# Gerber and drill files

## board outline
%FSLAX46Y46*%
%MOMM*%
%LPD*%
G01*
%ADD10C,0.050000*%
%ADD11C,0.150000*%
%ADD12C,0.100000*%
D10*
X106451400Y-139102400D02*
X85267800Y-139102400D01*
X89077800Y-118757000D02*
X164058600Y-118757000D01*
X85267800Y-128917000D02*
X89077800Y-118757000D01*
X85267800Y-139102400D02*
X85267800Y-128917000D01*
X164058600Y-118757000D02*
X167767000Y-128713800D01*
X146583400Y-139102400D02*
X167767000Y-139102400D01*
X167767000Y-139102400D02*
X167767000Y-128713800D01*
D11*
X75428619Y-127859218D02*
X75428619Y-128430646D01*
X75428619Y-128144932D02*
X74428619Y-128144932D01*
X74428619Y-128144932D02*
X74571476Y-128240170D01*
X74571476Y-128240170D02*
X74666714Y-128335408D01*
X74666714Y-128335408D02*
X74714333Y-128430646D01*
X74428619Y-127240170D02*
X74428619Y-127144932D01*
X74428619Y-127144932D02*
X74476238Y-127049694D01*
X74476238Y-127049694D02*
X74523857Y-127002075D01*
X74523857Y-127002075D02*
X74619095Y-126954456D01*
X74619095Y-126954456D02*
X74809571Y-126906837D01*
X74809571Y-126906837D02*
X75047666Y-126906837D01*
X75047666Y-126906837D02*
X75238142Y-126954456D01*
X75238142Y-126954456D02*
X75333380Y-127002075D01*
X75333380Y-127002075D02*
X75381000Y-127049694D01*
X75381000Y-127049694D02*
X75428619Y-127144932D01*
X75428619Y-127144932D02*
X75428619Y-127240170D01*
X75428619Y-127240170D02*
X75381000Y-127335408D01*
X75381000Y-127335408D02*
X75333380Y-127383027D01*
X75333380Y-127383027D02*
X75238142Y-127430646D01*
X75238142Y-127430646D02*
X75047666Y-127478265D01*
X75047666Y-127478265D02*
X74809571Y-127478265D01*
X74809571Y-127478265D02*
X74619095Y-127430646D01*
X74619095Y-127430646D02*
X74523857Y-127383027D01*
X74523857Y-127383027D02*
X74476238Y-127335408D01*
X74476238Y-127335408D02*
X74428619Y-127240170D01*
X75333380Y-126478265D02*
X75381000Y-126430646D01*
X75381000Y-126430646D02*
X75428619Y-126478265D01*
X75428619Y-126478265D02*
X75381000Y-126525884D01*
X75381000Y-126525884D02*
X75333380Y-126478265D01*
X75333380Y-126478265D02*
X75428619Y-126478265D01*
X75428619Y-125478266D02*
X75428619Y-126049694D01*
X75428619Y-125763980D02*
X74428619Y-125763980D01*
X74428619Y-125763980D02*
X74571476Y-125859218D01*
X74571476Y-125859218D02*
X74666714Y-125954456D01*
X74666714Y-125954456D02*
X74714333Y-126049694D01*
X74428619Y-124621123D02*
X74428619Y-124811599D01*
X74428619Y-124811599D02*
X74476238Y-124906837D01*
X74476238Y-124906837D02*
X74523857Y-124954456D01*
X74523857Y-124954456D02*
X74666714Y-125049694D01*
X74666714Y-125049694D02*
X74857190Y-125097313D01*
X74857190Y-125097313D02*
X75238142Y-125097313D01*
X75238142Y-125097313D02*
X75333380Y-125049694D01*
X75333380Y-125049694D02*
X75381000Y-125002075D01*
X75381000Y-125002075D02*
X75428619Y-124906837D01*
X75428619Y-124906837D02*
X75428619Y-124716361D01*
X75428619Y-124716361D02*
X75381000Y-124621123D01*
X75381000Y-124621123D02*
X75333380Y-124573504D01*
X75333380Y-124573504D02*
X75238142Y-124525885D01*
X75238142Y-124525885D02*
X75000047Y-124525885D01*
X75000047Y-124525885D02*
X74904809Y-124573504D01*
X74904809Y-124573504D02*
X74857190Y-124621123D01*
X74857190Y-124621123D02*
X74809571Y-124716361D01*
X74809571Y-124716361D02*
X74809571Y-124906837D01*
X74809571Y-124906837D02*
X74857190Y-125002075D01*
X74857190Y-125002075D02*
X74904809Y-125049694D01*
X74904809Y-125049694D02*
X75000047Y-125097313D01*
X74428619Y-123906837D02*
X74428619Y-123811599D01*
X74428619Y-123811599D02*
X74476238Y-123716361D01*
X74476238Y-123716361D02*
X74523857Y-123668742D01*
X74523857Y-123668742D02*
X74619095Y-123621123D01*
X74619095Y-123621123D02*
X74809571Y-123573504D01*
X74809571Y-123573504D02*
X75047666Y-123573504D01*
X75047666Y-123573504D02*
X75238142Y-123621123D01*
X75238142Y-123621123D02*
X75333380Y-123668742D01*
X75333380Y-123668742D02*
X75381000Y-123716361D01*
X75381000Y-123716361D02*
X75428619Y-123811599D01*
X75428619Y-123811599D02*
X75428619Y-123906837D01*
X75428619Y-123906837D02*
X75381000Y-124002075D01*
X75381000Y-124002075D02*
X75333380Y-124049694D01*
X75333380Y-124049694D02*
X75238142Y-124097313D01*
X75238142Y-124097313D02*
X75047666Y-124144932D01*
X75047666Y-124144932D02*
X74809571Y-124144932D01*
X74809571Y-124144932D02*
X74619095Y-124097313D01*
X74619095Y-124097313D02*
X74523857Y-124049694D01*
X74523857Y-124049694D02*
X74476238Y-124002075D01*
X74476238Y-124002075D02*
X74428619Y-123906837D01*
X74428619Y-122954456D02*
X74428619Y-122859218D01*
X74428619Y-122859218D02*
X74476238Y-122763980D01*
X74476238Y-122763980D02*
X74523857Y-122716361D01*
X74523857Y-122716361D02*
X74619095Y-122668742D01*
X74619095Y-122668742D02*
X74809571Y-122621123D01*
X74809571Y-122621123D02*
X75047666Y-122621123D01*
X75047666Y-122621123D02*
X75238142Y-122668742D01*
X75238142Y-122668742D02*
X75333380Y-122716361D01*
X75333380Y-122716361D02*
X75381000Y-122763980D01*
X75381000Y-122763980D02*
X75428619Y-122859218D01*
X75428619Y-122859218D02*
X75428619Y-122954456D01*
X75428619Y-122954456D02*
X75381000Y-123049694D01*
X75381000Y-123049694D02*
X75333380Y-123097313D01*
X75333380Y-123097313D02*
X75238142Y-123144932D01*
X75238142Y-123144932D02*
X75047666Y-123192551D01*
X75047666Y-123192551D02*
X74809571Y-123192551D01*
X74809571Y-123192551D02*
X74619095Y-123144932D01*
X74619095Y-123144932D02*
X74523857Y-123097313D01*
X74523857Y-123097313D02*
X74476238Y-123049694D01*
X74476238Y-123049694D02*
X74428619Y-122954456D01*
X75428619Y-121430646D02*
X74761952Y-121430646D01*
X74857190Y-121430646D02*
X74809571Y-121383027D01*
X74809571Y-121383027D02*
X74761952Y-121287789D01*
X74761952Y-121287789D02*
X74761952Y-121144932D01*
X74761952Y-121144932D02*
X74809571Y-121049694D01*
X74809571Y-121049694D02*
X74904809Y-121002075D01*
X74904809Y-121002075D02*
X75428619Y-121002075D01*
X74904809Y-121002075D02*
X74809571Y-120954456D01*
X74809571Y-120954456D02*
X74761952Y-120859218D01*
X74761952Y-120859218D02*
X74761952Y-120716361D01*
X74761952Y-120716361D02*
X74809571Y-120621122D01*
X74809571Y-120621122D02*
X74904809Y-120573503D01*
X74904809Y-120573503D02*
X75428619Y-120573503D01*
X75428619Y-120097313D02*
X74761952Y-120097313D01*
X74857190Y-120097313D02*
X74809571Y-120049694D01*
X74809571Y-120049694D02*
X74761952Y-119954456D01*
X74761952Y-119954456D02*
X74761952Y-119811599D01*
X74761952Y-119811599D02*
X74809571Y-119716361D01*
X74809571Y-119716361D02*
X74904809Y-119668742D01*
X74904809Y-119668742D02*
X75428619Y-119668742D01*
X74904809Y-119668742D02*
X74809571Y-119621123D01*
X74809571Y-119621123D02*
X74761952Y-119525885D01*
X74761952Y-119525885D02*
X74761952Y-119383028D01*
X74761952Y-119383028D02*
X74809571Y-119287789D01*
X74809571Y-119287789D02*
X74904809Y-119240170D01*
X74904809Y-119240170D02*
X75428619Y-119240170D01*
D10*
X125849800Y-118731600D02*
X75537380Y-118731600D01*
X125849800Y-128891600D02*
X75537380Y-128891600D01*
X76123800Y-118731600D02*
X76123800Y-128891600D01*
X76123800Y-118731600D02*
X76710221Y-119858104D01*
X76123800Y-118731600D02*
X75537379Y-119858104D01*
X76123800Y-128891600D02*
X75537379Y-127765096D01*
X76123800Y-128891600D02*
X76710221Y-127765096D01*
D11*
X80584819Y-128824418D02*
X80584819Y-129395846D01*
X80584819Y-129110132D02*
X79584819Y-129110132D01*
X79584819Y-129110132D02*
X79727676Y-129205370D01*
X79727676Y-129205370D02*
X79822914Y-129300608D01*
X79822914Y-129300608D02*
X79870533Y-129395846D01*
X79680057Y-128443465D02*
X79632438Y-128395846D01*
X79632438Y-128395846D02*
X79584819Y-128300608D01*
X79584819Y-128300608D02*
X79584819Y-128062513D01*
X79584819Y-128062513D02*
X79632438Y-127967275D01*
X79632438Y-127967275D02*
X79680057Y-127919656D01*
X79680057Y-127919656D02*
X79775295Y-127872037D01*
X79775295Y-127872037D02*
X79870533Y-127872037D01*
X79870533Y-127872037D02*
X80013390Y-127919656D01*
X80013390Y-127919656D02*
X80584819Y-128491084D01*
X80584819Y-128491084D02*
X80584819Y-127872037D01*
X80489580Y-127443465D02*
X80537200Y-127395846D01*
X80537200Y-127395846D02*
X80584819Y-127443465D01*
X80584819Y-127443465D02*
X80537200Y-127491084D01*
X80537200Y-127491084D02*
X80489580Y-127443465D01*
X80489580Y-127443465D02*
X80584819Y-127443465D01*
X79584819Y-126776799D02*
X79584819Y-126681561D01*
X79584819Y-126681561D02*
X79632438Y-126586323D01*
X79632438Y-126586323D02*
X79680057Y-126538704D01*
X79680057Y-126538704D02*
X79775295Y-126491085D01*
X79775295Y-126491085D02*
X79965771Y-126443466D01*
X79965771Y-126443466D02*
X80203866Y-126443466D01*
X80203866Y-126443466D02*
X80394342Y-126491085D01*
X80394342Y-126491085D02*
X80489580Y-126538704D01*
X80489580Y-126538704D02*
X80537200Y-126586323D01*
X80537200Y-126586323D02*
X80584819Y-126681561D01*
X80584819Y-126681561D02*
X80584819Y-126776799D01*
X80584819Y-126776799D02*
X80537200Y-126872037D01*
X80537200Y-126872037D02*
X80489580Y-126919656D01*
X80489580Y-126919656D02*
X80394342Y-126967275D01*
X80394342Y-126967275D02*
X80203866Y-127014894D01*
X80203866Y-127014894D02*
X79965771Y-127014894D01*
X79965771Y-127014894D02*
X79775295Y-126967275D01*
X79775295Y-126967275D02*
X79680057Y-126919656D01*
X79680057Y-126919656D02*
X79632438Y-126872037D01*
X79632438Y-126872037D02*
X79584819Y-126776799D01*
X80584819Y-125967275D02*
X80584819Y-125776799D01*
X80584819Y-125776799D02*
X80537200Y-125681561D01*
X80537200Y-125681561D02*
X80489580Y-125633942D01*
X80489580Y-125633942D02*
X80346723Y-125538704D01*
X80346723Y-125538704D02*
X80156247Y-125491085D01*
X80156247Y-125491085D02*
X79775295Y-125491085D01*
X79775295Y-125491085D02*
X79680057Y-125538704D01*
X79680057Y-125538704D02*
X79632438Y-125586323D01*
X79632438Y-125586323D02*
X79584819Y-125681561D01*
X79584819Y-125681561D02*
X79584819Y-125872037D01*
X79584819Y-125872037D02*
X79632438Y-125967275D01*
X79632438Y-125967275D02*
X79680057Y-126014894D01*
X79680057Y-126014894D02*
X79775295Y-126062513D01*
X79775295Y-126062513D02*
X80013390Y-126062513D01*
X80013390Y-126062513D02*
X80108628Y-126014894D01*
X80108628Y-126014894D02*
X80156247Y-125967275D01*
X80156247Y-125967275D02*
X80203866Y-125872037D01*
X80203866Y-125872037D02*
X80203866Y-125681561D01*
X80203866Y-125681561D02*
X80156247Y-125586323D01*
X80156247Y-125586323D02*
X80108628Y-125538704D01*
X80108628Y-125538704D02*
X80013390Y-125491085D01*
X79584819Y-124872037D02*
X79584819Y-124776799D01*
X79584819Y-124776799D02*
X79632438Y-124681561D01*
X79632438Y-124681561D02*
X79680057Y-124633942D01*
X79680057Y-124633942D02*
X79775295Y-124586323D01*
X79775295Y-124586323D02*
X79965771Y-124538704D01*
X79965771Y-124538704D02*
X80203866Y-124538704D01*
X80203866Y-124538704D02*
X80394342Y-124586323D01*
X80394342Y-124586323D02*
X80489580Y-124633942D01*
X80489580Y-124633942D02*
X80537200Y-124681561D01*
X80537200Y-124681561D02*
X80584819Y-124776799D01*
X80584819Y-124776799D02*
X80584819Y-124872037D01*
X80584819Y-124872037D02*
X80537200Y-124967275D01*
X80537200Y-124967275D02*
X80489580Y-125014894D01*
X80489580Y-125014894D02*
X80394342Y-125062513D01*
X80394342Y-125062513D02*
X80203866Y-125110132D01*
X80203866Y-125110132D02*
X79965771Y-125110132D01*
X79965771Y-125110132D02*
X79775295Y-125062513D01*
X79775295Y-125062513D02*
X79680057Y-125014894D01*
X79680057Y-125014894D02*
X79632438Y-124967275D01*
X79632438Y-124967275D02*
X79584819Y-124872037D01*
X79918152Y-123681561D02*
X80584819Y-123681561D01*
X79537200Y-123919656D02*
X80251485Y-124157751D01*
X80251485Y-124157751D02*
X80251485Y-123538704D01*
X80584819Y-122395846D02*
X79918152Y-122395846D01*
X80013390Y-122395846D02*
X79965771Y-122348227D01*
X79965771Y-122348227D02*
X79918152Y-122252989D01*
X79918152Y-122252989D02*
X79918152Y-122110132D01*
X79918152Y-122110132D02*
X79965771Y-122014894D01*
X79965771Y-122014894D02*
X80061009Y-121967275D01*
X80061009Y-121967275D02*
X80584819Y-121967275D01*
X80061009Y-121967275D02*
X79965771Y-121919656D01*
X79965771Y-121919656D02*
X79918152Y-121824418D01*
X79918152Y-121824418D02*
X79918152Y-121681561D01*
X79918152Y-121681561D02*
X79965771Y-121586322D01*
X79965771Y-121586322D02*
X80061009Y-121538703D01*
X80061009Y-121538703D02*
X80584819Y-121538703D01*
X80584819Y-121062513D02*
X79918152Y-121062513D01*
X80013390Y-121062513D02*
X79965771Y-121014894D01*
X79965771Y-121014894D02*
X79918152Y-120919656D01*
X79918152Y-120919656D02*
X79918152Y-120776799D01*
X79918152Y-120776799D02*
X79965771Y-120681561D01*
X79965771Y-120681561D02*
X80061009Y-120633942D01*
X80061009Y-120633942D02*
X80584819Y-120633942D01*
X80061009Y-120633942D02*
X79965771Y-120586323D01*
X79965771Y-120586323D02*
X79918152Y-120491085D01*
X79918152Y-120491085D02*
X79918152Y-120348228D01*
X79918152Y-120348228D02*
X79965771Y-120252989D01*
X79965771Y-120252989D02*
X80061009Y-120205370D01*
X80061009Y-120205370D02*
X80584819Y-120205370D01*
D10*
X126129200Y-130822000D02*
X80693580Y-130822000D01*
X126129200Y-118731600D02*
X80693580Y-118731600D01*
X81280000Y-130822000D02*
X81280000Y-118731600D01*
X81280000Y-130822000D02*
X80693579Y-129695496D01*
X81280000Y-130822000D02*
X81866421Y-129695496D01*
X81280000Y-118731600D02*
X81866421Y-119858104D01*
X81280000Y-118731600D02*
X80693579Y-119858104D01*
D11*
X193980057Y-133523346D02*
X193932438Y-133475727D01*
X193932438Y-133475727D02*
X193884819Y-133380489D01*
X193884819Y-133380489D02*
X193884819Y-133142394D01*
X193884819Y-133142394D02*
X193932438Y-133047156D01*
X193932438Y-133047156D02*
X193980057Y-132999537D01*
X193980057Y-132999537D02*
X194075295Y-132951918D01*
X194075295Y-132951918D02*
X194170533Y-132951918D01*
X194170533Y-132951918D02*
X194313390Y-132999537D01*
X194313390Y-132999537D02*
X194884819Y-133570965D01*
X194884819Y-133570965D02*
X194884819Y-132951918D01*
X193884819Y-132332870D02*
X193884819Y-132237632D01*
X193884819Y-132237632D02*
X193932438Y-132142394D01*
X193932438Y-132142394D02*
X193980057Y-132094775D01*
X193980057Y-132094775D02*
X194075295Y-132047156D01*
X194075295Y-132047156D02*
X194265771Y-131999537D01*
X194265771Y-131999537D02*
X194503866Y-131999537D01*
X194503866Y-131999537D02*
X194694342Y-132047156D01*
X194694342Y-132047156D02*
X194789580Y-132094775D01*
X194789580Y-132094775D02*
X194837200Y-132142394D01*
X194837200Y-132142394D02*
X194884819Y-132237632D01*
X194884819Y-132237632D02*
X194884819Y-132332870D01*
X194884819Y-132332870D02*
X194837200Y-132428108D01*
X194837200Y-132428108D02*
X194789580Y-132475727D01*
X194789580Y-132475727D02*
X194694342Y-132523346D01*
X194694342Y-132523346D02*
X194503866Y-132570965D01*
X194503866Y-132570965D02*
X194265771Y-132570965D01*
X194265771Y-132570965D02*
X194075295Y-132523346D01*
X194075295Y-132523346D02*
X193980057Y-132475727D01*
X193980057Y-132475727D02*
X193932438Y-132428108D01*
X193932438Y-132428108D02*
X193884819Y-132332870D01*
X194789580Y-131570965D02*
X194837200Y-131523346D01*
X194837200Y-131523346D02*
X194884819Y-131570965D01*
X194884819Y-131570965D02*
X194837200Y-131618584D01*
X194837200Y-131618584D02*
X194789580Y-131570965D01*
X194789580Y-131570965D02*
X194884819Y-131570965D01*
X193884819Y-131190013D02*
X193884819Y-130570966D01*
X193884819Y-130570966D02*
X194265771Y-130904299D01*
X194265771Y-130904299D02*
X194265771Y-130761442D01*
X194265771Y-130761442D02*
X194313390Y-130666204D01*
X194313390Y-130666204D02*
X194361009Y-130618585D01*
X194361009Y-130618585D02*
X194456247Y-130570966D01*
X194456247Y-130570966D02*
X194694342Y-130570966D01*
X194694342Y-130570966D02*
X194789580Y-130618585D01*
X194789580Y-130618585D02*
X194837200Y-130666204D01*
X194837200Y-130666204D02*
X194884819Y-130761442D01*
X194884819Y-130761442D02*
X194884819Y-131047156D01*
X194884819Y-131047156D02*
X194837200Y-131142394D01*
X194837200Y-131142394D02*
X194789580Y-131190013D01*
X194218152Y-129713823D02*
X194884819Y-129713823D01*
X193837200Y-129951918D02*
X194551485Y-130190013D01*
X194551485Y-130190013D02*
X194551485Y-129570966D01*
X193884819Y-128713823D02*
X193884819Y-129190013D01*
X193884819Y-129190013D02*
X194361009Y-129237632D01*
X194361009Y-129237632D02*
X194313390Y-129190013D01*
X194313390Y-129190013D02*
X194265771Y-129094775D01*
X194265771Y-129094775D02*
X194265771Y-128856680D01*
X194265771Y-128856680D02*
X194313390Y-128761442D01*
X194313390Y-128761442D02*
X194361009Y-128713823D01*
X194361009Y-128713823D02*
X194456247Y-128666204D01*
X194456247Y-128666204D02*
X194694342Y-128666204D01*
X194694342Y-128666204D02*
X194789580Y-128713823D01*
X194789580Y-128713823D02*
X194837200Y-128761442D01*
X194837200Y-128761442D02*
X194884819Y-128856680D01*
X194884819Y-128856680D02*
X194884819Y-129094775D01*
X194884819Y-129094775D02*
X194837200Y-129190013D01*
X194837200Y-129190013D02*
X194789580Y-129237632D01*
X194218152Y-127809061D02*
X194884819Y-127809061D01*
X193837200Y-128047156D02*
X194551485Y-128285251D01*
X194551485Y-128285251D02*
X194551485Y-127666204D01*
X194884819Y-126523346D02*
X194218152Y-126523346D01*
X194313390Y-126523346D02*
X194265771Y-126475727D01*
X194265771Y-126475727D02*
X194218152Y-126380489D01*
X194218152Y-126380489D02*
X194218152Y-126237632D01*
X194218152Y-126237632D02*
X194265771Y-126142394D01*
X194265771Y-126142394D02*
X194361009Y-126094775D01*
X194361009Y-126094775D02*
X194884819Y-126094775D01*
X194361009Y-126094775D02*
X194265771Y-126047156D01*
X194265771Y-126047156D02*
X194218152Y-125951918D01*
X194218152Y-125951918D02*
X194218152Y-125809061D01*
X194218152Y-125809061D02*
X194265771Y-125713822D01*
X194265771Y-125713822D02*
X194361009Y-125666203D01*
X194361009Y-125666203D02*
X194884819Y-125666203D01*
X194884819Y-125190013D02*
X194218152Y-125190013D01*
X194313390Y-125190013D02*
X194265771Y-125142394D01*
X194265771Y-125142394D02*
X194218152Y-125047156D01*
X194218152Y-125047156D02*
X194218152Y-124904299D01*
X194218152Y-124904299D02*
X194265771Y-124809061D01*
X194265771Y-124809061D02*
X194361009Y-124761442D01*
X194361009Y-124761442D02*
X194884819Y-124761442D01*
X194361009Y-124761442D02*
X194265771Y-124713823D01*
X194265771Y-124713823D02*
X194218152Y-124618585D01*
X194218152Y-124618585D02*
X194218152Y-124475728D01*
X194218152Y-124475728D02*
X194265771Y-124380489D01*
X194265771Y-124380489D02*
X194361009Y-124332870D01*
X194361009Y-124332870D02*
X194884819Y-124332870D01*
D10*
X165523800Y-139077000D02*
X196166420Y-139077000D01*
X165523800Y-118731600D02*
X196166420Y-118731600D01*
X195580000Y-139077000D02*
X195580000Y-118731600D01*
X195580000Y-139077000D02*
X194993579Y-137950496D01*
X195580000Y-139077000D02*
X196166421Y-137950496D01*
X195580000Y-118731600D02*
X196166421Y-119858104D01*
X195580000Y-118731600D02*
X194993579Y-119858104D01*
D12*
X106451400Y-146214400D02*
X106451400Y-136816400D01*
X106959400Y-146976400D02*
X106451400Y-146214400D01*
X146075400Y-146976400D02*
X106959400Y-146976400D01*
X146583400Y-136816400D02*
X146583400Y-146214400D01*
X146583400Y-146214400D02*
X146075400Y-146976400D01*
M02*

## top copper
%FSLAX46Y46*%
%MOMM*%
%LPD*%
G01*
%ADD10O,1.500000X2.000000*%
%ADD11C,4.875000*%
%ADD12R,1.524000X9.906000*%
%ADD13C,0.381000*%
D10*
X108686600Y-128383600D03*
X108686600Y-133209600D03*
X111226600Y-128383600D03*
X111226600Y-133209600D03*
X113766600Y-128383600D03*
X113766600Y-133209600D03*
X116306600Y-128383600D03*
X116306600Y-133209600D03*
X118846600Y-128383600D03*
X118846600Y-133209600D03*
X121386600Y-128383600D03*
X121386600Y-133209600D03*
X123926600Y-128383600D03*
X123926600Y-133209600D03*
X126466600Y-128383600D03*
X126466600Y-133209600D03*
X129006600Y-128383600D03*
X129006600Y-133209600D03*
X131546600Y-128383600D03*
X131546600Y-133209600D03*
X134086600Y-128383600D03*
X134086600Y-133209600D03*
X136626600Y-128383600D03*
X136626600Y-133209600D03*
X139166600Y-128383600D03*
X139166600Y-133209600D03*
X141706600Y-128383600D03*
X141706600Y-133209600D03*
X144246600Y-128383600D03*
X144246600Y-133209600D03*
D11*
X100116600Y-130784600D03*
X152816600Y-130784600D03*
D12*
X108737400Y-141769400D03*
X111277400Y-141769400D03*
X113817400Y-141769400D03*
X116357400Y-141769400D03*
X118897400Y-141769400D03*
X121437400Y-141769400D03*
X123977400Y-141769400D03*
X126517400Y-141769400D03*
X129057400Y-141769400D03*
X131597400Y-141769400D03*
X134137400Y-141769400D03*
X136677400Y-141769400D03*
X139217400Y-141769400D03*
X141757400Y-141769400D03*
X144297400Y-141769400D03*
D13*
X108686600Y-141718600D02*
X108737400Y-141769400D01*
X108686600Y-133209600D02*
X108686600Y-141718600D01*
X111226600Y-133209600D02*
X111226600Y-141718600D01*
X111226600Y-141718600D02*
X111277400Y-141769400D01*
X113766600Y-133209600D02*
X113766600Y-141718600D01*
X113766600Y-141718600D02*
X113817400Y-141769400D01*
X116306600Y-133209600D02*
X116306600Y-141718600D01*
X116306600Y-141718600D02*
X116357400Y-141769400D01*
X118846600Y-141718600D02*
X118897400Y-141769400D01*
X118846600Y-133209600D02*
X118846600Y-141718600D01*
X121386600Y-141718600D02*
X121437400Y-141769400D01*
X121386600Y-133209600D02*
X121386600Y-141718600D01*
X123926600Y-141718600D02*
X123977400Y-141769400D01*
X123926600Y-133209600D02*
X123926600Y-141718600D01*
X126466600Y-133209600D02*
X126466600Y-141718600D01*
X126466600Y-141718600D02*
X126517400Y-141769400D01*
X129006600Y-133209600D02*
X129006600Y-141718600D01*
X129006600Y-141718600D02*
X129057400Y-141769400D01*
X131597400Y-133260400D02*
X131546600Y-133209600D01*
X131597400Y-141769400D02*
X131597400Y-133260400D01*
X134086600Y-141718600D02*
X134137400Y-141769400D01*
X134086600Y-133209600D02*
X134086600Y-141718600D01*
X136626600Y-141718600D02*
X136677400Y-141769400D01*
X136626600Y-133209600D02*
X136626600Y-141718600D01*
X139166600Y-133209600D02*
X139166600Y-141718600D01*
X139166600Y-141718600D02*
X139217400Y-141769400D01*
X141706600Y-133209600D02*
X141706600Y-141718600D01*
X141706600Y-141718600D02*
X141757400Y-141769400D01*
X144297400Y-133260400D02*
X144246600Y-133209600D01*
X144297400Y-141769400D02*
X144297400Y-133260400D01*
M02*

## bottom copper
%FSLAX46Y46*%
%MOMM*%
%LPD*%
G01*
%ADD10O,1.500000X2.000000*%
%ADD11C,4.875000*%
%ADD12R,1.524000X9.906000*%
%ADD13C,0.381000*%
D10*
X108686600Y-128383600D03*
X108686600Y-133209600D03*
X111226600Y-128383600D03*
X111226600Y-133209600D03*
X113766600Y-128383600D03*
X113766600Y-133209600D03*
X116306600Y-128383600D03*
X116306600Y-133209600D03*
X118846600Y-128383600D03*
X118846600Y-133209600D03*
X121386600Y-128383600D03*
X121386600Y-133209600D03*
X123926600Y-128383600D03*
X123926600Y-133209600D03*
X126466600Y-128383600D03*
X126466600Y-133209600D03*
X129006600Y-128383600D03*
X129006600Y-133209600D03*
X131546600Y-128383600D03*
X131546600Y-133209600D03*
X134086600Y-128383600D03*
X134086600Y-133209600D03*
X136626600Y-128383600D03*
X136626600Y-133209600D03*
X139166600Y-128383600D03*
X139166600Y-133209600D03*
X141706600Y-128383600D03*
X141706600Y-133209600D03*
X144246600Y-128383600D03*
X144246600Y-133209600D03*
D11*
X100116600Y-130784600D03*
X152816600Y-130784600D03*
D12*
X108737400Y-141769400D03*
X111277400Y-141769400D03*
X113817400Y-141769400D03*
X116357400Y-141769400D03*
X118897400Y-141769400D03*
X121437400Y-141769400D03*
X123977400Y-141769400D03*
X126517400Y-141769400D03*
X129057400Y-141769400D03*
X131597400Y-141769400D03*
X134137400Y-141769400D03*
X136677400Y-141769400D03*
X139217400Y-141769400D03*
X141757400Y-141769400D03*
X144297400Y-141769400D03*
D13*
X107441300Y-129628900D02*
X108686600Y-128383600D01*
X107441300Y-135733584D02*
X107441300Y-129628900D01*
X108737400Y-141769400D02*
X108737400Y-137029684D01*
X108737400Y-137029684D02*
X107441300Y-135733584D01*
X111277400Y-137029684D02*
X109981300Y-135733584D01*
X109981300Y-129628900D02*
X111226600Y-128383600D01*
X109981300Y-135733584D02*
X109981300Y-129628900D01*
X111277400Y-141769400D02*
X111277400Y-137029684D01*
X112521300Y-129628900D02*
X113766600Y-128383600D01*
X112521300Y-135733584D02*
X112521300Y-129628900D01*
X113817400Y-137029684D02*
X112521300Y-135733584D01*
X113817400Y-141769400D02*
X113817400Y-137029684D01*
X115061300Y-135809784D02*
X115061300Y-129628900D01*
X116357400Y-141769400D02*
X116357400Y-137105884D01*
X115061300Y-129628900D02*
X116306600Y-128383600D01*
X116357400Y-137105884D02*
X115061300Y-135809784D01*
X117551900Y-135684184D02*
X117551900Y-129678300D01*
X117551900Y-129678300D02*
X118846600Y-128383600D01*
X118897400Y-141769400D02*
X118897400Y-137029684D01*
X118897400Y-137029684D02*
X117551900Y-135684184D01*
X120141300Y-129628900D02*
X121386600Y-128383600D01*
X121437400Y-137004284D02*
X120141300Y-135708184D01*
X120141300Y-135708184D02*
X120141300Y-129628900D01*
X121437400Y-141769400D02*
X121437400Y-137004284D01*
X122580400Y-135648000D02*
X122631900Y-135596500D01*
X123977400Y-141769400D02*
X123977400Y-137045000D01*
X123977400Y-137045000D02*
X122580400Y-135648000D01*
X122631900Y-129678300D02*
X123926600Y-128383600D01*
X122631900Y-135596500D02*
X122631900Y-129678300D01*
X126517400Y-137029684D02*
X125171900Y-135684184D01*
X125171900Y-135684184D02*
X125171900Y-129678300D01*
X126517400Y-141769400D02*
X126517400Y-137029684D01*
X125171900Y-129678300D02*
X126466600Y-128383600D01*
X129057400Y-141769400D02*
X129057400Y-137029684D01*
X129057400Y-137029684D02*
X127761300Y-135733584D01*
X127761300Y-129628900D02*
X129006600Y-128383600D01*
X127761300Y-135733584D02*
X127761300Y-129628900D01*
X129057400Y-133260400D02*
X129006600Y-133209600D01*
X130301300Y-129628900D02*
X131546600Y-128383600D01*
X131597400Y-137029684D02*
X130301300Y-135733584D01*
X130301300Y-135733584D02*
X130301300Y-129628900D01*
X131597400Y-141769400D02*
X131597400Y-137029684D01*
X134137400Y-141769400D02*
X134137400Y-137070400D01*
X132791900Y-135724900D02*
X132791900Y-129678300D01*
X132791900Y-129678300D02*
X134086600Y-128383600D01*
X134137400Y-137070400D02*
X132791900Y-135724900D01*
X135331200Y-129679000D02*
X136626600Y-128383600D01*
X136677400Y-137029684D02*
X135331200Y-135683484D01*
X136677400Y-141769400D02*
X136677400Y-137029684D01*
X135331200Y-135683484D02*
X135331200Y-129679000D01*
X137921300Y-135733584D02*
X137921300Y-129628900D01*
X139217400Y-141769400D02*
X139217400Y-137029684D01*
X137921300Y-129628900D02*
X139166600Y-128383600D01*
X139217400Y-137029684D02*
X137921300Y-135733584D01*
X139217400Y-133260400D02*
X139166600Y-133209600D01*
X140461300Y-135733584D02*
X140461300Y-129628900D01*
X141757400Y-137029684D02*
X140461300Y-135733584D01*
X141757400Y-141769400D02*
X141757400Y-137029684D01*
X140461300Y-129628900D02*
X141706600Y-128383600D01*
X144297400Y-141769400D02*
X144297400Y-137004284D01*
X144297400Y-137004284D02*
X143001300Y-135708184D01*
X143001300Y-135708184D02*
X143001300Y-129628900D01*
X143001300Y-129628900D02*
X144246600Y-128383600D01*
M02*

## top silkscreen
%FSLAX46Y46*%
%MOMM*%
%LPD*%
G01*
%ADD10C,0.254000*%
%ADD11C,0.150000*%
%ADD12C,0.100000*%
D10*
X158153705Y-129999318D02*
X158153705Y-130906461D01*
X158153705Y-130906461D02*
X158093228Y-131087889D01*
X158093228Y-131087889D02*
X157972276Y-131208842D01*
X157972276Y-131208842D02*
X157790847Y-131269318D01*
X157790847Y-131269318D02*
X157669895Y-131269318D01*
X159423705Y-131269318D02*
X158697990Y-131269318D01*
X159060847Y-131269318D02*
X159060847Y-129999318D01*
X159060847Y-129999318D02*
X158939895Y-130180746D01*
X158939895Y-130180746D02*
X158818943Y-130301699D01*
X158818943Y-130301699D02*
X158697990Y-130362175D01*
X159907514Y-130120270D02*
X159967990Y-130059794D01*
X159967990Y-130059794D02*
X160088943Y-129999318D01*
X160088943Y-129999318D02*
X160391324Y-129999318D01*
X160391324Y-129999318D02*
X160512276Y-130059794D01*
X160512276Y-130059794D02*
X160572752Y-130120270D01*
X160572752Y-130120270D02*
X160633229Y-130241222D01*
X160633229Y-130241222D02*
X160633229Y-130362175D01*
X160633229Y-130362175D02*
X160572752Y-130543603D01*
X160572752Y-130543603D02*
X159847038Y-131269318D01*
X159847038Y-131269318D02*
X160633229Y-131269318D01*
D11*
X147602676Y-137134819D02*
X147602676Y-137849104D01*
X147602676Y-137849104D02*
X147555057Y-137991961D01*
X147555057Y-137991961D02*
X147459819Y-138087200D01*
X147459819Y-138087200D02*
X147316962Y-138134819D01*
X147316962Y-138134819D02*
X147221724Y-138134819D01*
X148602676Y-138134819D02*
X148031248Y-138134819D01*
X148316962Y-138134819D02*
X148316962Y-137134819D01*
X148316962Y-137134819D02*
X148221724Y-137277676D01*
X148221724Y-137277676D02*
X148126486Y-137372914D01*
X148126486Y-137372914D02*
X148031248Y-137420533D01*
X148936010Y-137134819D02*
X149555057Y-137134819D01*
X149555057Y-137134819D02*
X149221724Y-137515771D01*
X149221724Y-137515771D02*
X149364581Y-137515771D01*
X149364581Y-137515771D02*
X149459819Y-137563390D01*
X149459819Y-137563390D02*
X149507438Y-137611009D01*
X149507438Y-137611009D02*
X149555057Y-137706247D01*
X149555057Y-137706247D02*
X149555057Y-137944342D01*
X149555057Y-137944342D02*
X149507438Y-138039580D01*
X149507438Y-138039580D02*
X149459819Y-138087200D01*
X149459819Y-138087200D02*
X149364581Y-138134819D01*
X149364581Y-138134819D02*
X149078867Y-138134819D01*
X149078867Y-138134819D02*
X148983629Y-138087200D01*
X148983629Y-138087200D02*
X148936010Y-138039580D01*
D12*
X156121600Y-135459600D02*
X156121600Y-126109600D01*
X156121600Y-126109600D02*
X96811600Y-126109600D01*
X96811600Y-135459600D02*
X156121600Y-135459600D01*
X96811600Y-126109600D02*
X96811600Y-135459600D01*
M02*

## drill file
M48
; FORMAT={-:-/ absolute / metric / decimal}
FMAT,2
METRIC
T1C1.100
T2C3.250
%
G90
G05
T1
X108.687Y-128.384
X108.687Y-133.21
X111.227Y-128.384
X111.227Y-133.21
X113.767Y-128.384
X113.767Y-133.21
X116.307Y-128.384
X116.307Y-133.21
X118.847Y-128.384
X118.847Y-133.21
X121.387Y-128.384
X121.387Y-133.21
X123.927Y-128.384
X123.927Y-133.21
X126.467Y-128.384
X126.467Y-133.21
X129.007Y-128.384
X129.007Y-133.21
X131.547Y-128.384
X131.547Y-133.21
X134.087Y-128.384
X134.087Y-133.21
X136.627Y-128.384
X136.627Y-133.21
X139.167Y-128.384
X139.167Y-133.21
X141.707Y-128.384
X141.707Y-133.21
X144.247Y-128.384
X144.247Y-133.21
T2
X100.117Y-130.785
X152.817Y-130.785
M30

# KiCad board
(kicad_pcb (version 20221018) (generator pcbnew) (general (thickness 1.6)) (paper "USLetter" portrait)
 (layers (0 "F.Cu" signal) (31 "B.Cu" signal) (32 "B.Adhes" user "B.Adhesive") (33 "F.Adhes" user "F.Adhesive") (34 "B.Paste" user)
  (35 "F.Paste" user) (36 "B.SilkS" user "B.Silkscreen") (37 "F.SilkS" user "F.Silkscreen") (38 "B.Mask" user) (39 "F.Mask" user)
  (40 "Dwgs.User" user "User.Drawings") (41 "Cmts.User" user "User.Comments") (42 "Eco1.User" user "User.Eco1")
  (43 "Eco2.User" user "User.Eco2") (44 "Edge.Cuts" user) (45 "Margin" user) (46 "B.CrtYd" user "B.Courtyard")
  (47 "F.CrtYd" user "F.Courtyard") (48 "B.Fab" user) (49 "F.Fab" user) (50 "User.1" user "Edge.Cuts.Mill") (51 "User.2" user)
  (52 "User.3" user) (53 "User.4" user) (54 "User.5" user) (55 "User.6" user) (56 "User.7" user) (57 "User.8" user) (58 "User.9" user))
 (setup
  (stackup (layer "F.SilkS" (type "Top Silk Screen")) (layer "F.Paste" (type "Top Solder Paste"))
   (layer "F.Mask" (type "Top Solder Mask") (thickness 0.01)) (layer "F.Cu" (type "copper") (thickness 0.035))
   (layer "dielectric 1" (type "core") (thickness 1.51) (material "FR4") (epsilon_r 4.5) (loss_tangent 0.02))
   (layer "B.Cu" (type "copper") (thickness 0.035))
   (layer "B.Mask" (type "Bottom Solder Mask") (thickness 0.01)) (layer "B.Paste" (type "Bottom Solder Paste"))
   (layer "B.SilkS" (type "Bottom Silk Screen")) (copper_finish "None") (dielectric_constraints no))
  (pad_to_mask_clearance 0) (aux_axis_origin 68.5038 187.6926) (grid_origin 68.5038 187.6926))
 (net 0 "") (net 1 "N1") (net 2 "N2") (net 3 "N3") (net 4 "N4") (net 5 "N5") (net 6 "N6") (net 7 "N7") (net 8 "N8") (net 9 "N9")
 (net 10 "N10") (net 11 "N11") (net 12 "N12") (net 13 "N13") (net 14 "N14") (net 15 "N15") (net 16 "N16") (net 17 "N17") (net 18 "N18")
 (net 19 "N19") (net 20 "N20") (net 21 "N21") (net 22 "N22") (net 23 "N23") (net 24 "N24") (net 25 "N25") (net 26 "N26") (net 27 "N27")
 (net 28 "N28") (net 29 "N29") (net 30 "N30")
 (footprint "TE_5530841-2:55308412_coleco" (layer "F.Cu") (at 108.6866 133.2096 180)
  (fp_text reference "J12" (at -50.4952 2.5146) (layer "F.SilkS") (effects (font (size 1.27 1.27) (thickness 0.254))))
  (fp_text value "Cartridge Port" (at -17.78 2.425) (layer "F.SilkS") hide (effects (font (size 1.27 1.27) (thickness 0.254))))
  (fp_line (start -47.435 -2.25) (end -47.435 7.1) (stroke (width 0.1) (type solid)) (layer "F.SilkS"))
  (fp_line (start -47.435 7.1) (end 11.875 7.1) (stroke (width 0.1) (type solid)) (layer "F.SilkS"))
  (fp_line (start 11.875 -2.25) (end -47.435 -2.25) (stroke (width 0.1) (type solid)) (layer "F.SilkS"))
  (fp_line (start 11.875 7.1) (end 11.875 -2.25) (stroke (width 0.1) (type solid)) (layer "F.SilkS"))
  (pad "1" thru_hole oval (at 0 4.826 180) (size 1.5 2) (drill 1.1) (layers "*.Cu" "*.Mask") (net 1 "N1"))
  (pad "2" thru_hole oval (at 0 0 180) (size 1.5 2) (drill 1.1) (layers "*.Cu" "*.Mask") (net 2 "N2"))
  (pad "3" thru_hole oval (at -2.54 4.826 180) (size 1.5 2) (drill 1.1) (layers "*.Cu" "*.Mask") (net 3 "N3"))
  (pad "4" thru_hole oval (at -2.54 0 180) (size 1.5 2) (drill 1.1) (layers "*.Cu" "*.Mask") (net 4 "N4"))
  (pad "5" thru_hole oval (at -5.08 4.826 180) (size 1.5 2) (drill 1.1) (layers "*.Cu" "*.Mask") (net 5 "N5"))
  (pad "6" thru_hole oval (at -5.08 0 180) (size 1.5 2) (drill 1.1) (layers "*.Cu" "*.Mask") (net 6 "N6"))
  (pad "7" thru_hole oval (at -7.62 4.826 180) (size 1.5 2) (drill 1.1) (layers "*.Cu" "*.Mask") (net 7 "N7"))
  (pad "8" thru_hole oval (at -7.62 0 180) (size 1.5 2) (drill 1.1) (layers "*.Cu" "*.Mask") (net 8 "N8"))
  (pad "9" thru_hole oval (at -10.16 4.826 180) (size 1.5 2) (drill 1.1) (layers "*.Cu" "*.Mask") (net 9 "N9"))
  (pad "10" thru_hole oval (at -10.16 0 180) (size 1.5 2) (drill 1.1) (layers "*.Cu" "*.Mask") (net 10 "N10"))
  (pad "11" thru_hole oval (at -12.7 4.826 180) (size 1.5 2) (drill 1.1) (layers "*.Cu" "*.Mask") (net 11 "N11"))
  (pad "12" thru_hole oval (at -12.7 0 180) (size 1.5 2) (drill 1.1) (layers "*.Cu" "*.Mask") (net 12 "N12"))
  (pad "13" thru_hole oval (at -15.24 4.826 180) (size 1.5 2) (drill 1.1) (layers "*.Cu" "*.Mask") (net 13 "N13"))
  (pad "14" thru_hole oval (at -15.24 0 180) (size 1.5 2) (drill 1.1) (layers "*.Cu" "*.Mask") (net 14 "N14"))
  (pad "15" thru_hole oval (at -17.78 4.826 180) (size 1.5 2) (drill 1.1) (layers "*.Cu" "*.Mask") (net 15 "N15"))
  (pad "16" thru_hole oval (at -17.78 0 180) (size 1.5 2) (drill 1.1) (layers "*.Cu" "*.Mask") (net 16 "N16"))
  (pad "17" thru_hole oval (at -20.32 4.826 180) (size 1.5 2) (drill 1.1) (layers "*.Cu" "*.Mask") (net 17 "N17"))
  (pad "18" thru_hole oval (at -20.32 0 180) (size 1.5 2) (drill 1.1) (layers "*.Cu" "*.Mask") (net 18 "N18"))
  (pad "19" thru_hole oval (at -22.86 4.826 180) (size 1.5 2) (drill 1.1) (layers "*.Cu" "*.Mask") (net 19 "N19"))
  (pad "20" thru_hole oval (at -22.86 0 180) (size 1.5 2) (drill 1.1) (layers "*.Cu" "*.Mask") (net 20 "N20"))
  (pad "21" thru_hole oval (at -25.4 4.826 180) (size 1.5 2) (drill 1.1) (layers "*.Cu" "*.Mask") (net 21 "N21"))
  (pad "22" thru_hole oval (at -25.4 0 180) (size 1.5 2) (drill 1.1) (layers "*.Cu" "*.Mask") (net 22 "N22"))
  (pad "23" thru_hole oval (at -27.94 4.826 180) (size 1.5 2) (drill 1.1) (layers "*.Cu" "*.Mask") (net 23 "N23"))
  (pad "24" thru_hole oval (at -27.94 0 180) (size 1.5 2) (drill 1.1) (layers "*.Cu" "*.Mask") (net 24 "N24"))
  (pad "25" thru_hole oval (at -30.48 4.826 180) (size 1.5 2) (drill 1.1) (layers "*.Cu" "*.Mask") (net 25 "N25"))
  (pad "26" thru_hole oval (at -30.48 0 180) (size 1.5 2) (drill 1.1) (layers "*.Cu" "*.Mask") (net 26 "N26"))
  (pad "27" thru_hole oval (at -33.02 4.826 180) (size 1.5 2) (drill 1.1) (layers "*.Cu" "*.Mask") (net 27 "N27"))
  (pad "28" thru_hole oval (at -33.02 0 180) (size 1.5 2) (drill 1.1) (layers "*.Cu" "*.Mask") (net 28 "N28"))
  (pad "29" thru_hole oval (at -35.56 4.826 180) (size 1.5 2) (drill 1.1) (layers "*.Cu" "*.Mask") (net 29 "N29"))
  (pad "30" thru_hole oval (at -35.56 0 180) (size 1.5 2) (drill 1.1) (layers "*.Cu" "*.Mask") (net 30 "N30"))
  (pad "MH1" thru_hole circle (at 8.57 2.425 180) (size 4.875 4.875) (drill 3.25) (layers "*.Cu" "*.Mask"))
  (pad "MH2" thru_hole circle (at -44.13 2.425 180) (size 4.875 4.875) (drill 3.25) (layers "*.Cu" "*.Mask")))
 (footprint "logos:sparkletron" (layer "F.Cu") (at 138.3842 226.960062)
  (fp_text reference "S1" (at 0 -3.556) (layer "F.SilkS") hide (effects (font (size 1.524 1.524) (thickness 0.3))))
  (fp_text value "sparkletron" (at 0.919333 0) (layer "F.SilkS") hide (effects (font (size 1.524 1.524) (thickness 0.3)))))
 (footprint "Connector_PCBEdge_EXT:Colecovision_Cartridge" (layer "F.Cu") (at 104.9274 143.6744)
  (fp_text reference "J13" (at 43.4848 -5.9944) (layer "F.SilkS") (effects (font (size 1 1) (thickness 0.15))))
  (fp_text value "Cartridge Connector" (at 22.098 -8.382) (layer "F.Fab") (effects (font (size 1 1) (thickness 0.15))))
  (fp_line (start 1.524 2.54) (end 1.524 -6.858) (stroke (width 0.1) (type solid)) (layer "Edge.Cuts"))
  (fp_line (start 2.032 3.302) (end 1.524 2.54) (stroke (width 0.1) (type solid)) (layer "Edge.Cuts"))
  (fp_line (start 41.148 3.302) (end 2.032 3.302) (stroke (width 0.1) (type solid)) (layer "Edge.Cuts"))
  (fp_line (start 41.656 -6.858) (end 41.656 2.54) (stroke (width 0.1) (type solid)) (layer "Edge.Cuts"))
  (fp_line (start 41.656 2.54) (end 41.148 3.302) (stroke (width 0.1) (type solid)) (layer "Edge.Cuts"))
  (pad "1" connect rect (at 3.81 -1.905) (size 1.524 9.906) (layers "B.Cu" "B.Mask") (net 1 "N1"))
  (pad "2" connect rect (at 3.81 -1.905) (size 1.524 9.906) (layers "F.Cu" "F.Mask") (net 2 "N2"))
  (pad "3" connect rect (at 6.35 -1.905) (size 1.524 9.906) (layers "B.Cu" "B.Mask") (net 3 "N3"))
  (pad "4" connect rect (at 6.35 -1.905) (size 1.524 9.906) (layers "F.Cu" "F.Mask") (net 4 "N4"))
  (pad "5" connect rect (at 8.89 -1.905) (size 1.524 9.906) (layers "B.Cu" "B.Mask") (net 5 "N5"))
  (pad "6" connect rect (at 8.89 -1.905) (size 1.524 9.906) (layers "F.Cu" "F.Mask") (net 6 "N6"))
  (pad "7" connect rect (at 11.43 -1.905) (size 1.524 9.906) (layers "B.Cu" "B.Mask") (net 7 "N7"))
  (pad "8" connect rect (at 11.43 -1.905) (size 1.524 9.906) (layers "F.Cu" "F.Mask") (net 8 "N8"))
  (pad "9" connect rect (at 13.97 -1.905) (size 1.524 9.906) (layers "B.Cu" "B.Mask") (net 9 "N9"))
  (pad "10" connect rect (at 13.97 -1.905) (size 1.524 9.906) (layers "F.Cu" "F.Mask") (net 10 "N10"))
  (pad "11" connect rect (at 16.51 -1.905) (size 1.524 9.906) (layers "B.Cu" "B.Mask") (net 11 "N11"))
  (pad "12" connect rect (at 16.51 -1.905) (size 1.524 9.906) (layers "F.Cu" "F.Mask") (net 12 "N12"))
  (pad "13" connect rect (at 19.05 -1.905) (size 1.524 9.906) (layers "B.Cu" "B.Mask") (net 13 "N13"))
  (pad "14" connect rect (at 19.05 -1.905) (size 1.524 9.906) (layers "F.Cu" "F.Mask") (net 14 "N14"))
  (pad "15" connect rect (at 21.59 -1.905) (size 1.524 9.906) (layers "B.Cu" "B.Mask") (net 15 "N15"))
  (pad "16" connect rect (at 21.59 -1.905) (size 1.524 9.906) (layers "F.Cu" "F.Mask") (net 16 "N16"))
  (pad "17" connect rect (at 24.13 -1.905) (size 1.524 9.906) (layers "B.Cu" "B.Mask") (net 17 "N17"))
  (pad "18" connect rect (at 24.13 -1.905) (size 1.524 9.906) (layers "F.Cu" "F.Mask") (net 18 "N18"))
  (pad "19" connect rect (at 26.67 -1.905) (size 1.524 9.906) (layers "B.Cu" "B.Mask") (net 19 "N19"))
  (pad "20" connect rect (at 26.67 -1.905) (size 1.524 9.906) (layers "F.Cu" "F.Mask") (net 20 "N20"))
  (pad "21" connect rect (at 29.21 -1.905) (size 1.524 9.906) (layers "B.Cu" "B.Mask") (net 21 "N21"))
  (pad "22" connect rect (at 29.21 -1.905) (size 1.524 9.906) (layers "F.Cu" "F.Mask") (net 22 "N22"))
  (pad "23" connect rect (at 31.75 -1.905) (size 1.524 9.906) (layers "B.Cu" "B.Mask") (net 23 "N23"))
  (pad "24" connect rect (at 31.75 -1.905) (size 1.524 9.906) (layers "F.Cu" "F.Mask") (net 24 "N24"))
  (pad "25" connect rect (at 34.29 -1.905) (size 1.524 9.906) (layers "B.Cu" "B.Mask") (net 25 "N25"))
  (pad "26" connect rect (at 34.29 -1.905) (size 1.524 9.906) (layers "F.Cu" "F.Mask") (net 26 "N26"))
  (pad "27" connect rect (at 36.83 -1.905) (size 1.524 9.906) (layers "B.Cu" "B.Mask") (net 27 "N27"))
  (pad "28" connect rect (at 36.83 -1.905) (size 1.524 9.906) (layers "F.Cu" "F.Mask") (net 28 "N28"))
  (pad "29" connect rect (at 39.37 -1.905) (size 1.524 9.906) (layers "B.Cu" "B.Mask") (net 29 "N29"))
  (pad "30" connect rect (at 39.37 -1.905) (size 1.524 9.906) (layers "F.Cu" "F.Mask") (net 30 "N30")))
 (gr_line (start 106.4514 139.1024) (end 85.2678 139.1024) (stroke (width 0.05) (type default)) (layer "Edge.Cuts"))
 (gr_line (start 89.0778 118.757) (end 164.0586 118.757) (stroke (width 0.05) (type default)) (layer "Edge.Cuts"))
 (gr_line (start 85.2678 128.917) (end 89.0778 118.757) (stroke (width 0.05) (type default)) (layer "Edge.Cuts"))
 (gr_line (start 85.2678 139.1024) (end 85.2678 128.917) (stroke (width 0.05) (type default)) (layer "Edge.Cuts"))
 (gr_line (start 164.0586 118.757) (end 167.767 128.7138) (stroke (width 0.05) (type default)) (layer "Edge.Cuts"))
 (gr_line (start 146.5834 139.1024) (end 167.767 139.1024) (stroke (width 0.05) (type default)) (layer "Edge.Cuts"))
 (gr_line (start 167.767 139.1024) (end 167.767 128.7138) (stroke (width 0.05) (type default)) (layer "Edge.Cuts"))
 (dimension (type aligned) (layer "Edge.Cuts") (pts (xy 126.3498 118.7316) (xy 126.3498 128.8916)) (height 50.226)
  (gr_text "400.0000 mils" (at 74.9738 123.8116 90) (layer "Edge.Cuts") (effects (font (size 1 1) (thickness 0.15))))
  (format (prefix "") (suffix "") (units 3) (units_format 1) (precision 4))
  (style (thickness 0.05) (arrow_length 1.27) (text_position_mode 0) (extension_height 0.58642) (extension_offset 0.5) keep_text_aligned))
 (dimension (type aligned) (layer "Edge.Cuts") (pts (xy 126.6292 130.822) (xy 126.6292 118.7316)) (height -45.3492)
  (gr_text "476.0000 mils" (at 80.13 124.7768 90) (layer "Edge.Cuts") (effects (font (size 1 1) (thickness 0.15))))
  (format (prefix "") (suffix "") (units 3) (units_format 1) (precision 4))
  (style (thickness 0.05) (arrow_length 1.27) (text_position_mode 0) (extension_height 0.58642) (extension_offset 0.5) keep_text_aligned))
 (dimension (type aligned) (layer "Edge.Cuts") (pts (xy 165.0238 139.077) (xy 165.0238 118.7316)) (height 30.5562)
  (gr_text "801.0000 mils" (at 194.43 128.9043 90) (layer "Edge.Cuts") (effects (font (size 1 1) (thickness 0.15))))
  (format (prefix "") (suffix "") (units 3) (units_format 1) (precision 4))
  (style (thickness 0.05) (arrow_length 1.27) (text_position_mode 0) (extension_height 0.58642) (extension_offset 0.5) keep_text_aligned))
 (segment (start 107.4413 129.6289) (end 108.6866 128.3836) (width 0.381) (layer "B.Cu") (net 1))
 (segment (start 107.4413 135.733584) (end 107.4413 129.6289) (width 0.381) (layer "B.Cu") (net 1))
 (segment (start 108.7374 141.7694) (end 108.7374 137.029684) (width 0.381) (layer "B.Cu") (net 1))
 (segment (start 108.7374 137.029684) (end 107.4413 135.733584) (width 0.381) (layer "B.Cu") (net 1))
 (segment (start 108.6866 141.7186) (end 108.7374 141.7694) (width 0.381) (layer "F.Cu") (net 2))
 (segment (start 108.6866 133.2096) (end 108.6866 141.7186) (width 0.381) (layer "F.Cu") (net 2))
 (segment (start 111.2774 137.029684) (end 109.9813 135.733584) (width 0.381) (layer "B.Cu") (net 3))
 (segment (start 109.9813 129.6289) (end 111.2266 128.3836) (width 0.381) (layer "B.Cu") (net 3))
 (segment (start 109.9813 135.733584) (end 109.9813 129.6289) (width 0.381) (layer "B.Cu") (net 3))
 (segment (start 111.2774 141.7694) (end 111.2774 137.029684) (width 0.381) (layer "B.Cu") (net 3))
 (segment (start 111.2266 133.2096) (end 111.2266 141.7186) (width 0.381) (layer "F.Cu") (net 4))
 (segment (start 111.2266 141.7186) (end 111.2774 141.7694) (width 0.381) (layer "F.Cu") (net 4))
 (segment (start 112.5213 129.6289) (end 113.7666 128.3836) (width 0.381) (layer "B.Cu") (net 5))
 (segment (start 112.5213 135.733584) (end 112.5213 129.6289) (width 0.381) (layer "B.Cu") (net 5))
 (segment (start 113.8174 137.029684) (end 112.5213 135.733584) (width 0.381) (layer "B.Cu") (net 5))
 (segment (start 113.8174 141.7694) (end 113.8174 137.029684) (width 0.381) (layer "B.Cu") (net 5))
 (segment (start 113.7666 133.2096) (end 113.7666 141.7186) (width 0.381) (layer "F.Cu") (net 6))
 (segment (start 113.7666 141.7186) (end 113.8174 141.7694) (width 0.381) (layer "F.Cu") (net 6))
 (segment (start 115.0613 135.809784) (end 115.0613 129.6289) (width 0.381) (layer "B.Cu") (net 7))
 (segment (start 116.3574 141.7694) (end 116.3574 137.105884) (width 0.381) (layer "B.Cu") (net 7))
 (segment (start 115.0613 129.6289) (end 116.3066 128.3836) (width 0.381) (layer "B.Cu") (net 7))
 (segment (start 116.3574 137.105884) (end 115.0613 135.809784) (width 0.381) (layer "B.Cu") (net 7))
 (segment (start 116.3066 133.2096) (end 116.3066 141.7186) (width 0.381) (layer "F.Cu") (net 8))
 (segment (start 116.3066 141.7186) (end 116.3574 141.7694) (width 0.381) (layer "F.Cu") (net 8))
 (segment (start 117.5519 135.684184) (end 117.5519 129.6783) (width 0.381) (layer "B.Cu") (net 9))
 (segment (start 117.5519 129.6783) (end 118.8466 128.3836) (width 0.381) (layer "B.Cu") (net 9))
 (segment (start 118.8974 141.7694) (end 118.8974 137.029684) (width 0.381) (layer "B.Cu") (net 9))
 (segment (start 118.8974 137.029684) (end 117.5519 135.684184) (width 0.381) (layer "B.Cu") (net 9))
 (segment (start 118.8466 141.7186) (end 118.8974 141.7694) (width 0.381) (layer "F.Cu") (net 10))
 (segment (start 118.8466 133.2096) (end 118.8466 141.7186) (width 0.381) (layer "F.Cu") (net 10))
 (segment (start 120.1413 129.6289) (end 121.3866 128.3836) (width 0.381) (layer "B.Cu") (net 11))
 (segment (start 121.4374 137.004284) (end 120.1413 135.708184) (width 0.381) (layer "B.Cu") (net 11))
 (segment (start 120.1413 135.708184) (end 120.1413 129.6289) (width 0.381) (layer "B.Cu") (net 11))
 (segment (start 121.4374 141.7694) (end 121.4374 137.004284) (width 0.381) (layer "B.Cu") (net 11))
 (segment (start 121.3866 141.7186) (end 121.4374 141.7694) (width 0.381) (layer "F.Cu") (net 12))
 (segment (start 121.3866 133.2096) (end 121.3866 141.7186) (width 0.381) (layer "F.Cu") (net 12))
 (segment (start 122.5804 135.648) (end 122.6319 135.5965) (width 0.381) (layer "B.Cu") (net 13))
 (segment (start 123.9774 141.7694) (end 123.9774 137.045) (width 0.381) (layer "B.Cu") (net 13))
 (segment (start 123.9774 137.045) (end 122.5804 135.648) (width 0.381) (layer "B.Cu") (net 13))
 (segment (start 122.6319 129.6783) (end 123.9266 128.3836) (width 0.381) (layer "B.Cu") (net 13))
 (segment (start 122.6319 135.5965) (end 122.6319 129.6783) (width 0.381) (layer "B.Cu") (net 13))
 (segment (start 123.9266 141.7186) (end 123.9774 141.7694) (width 0.381) (layer "F.Cu") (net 14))
 (segment (start 123.9266 133.2096) (end 123.9266 141.7186) (width 0.381) (layer "F.Cu") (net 14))
 (segment (start 126.5174 137.029684) (end 125.1719 135.684184) (width 0.381) (layer "B.Cu") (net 15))
 (segment (start 125.1719 135.684184) (end 125.1719 129.6783) (width 0.381) (layer "B.Cu") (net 15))
 (segment (start 126.5174 141.7694) (end 126.5174 137.029684) (width 0.381) (layer "B.Cu") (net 15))
 (segment (start 125.1719 129.6783) (end 126.4666 128.3836) (width 0.381) (layer "B.Cu") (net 15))
 (segment (start 126.4666 133.2096) (end 126.4666 141.7186) (width 0.381) (layer "F.Cu") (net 16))
 (segment (start 126.4666 141.7186) (end 126.5174 141.7694) (width 0.381) (layer "F.Cu") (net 16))
 (segment (start 129.0574 141.7694) (end 129.0574 137.029684) (width 0.381) (layer "B.Cu") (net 17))
 (segment (start 129.0574 137.029684) (end 127.7613 135.733584) (width 0.381) (layer "B.Cu") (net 17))
 (segment (start 127.7613 129.6289) (end 129.0066 128.3836) (width 0.381) (layer "B.Cu") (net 17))
 (segment (start 127.7613 135.733584) (end 127.7613 129.6289) (width 0.381) (layer "B.Cu") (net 17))
 (segment (start 129.0066 133.2096) (end 129.0066 141.7186) (width 0.381) (layer "F.Cu") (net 18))
 (segment (start 129.0066 141.7186) (end 129.0574 141.7694) (width 0.381) (layer "F.Cu") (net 18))
 (segment (start 129.0574 133.2604) (end 129.0066 133.2096) (width 0.381) (layer "B.Cu") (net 18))
 (segment (start 130.3013 129.6289) (end 131.5466 128.3836) (width 0.381) (layer "B.Cu") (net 19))
 (segment (start 131.5974 137.029684) (end 130.3013 135.733584) (width 0.381) (layer "B.Cu") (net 19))
 (segment (start 130.3013 135.733584) (end 130.3013 129.6289) (width 0.381) (layer "B.Cu") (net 19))
 (segment (start 131.5974 141.7694) (end 131.5974 137.029684) (width 0.381) (layer "B.Cu") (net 19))
 (segment (start 131.5974 133.2604) (end 131.5466 133.2096) (width 0.381) (layer "F.Cu") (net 20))
 (segment (start 131.5974 141.7694) (end 131.5974 133.2604) (width 0.381) (layer "F.Cu") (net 20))
 (segment (start 134.1374 141.7694) (end 134.1374 137.0704) (width 0.381) (layer "B.Cu") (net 21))
 (segment (start 132.7919 135.7249) (end 132.7919 129.6783) (width 0.381) (layer "B.Cu") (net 21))
 (segment (start 132.7919 129.6783) (end 134.0866 128.3836) (width 0.381) (layer "B.Cu") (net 21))
 (segment (start 134.1374 137.0704) (end 132.7919 135.7249) (width 0.381) (layer "B.Cu") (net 21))
 (segment (start 134.0866 141.7186) (end 134.1374 141.7694) (width 0.381) (layer "F.Cu") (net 22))
 (segment (start 134.0866 133.2096) (end 134.0866 141.7186) (width 0.381) (layer "F.Cu") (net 22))
 (segment (start 135.3312 129.679) (end 136.6266 128.3836) (width 0.381) (layer "B.Cu") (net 23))
 (segment (start 136.6774 137.029684) (end 135.3312 135.683484) (width 0.381) (layer "B.Cu") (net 23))
 (segment (start 136.6774 141.7694) (end 136.6774 137.029684) (width 0.381) (layer "B.Cu") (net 23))
 (segment (start 135.3312 135.683484) (end 135.3312 129.679) (width 0.381) (layer "B.Cu") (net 23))
 (segment (start 136.6266 141.7186) (end 136.6774 141.7694) (width 0.381) (layer "F.Cu") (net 24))
 (segment (start 136.6266 133.2096) (end 136.6266 141.7186) (width 0.381) (layer "F.Cu") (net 24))
 (segment (start 137.9213 135.733584) (end 137.9213 129.6289) (width 0.381) (layer "B.Cu") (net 25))
 (segment (start 139.2174 141.7694) (end 139.2174 137.029684) (width 0.381) (layer "B.Cu") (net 25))
 (segment (start 137.9213 129.6289) (end 139.1666 128.3836) (width 0.381) (layer "B.Cu") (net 25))
 (segment (start 139.2174 137.029684) (end 137.9213 135.733584) (width 0.381) (layer "B.Cu") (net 25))
 (segment (start 139.1666 133.2096) (end 139.1666 141.7186) (width 0.381) (layer "F.Cu") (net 26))
 (segment (start 139.1666 141.7186) (end 139.2174 141.7694) (width 0.381) (layer "F.Cu") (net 26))
 (segment (start 139.2174 133.2604) (end 139.1666 133.2096) (width 0.381) (layer "B.Cu") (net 26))
 (segment (start 140.4613 135.733584) (end 140.4613 129.6289) (width 0.381) (layer "B.Cu") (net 27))
 (segment (start 141.7574 137.029684) (end 140.4613 135.733584) (width 0.381) (layer "B.Cu") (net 27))
 (segment (start 141.7574 141.7694) (end 141.7574 137.029684) (width 0.381) (layer "B.Cu") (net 27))
 (segment (start 140.4613 129.6289) (end 141.7066 128.3836) (width 0.381) (layer "B.Cu") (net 27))
 (segment (start 141.7066 133.2096) (end 141.7066 141.7186) (width 0.381) (layer "F.Cu") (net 28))
 (segment (start 141.7066 141.7186) (end 141.7574 141.7694) (width 0.381) (layer "F.Cu") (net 28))
 (segment (start 144.2974 141.7694) (end 144.2974 137.004284) (width 0.381) (layer "B.Cu") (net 29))
 (segment (start 144.2974 137.004284) (end 143.0013 135.708184) (width 0.381) (layer "B.Cu") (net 29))
 (segment (start 143.0013 135.708184) (end 143.0013 129.6289) (width 0.381) (layer "B.Cu") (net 29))
 (segment (start 143.0013 129.6289) (end 144.2466 128.3836) (width 0.381) (layer "B.Cu") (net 29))
 (segment (start 144.2974 133.2604) (end 144.2466 133.2096) (width 0.381) (layer "F.Cu") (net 30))
 (segment (start 144.2974 141.7694) (end 144.2974 133.2604) (width 0.381) (layer "F.Cu") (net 30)))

